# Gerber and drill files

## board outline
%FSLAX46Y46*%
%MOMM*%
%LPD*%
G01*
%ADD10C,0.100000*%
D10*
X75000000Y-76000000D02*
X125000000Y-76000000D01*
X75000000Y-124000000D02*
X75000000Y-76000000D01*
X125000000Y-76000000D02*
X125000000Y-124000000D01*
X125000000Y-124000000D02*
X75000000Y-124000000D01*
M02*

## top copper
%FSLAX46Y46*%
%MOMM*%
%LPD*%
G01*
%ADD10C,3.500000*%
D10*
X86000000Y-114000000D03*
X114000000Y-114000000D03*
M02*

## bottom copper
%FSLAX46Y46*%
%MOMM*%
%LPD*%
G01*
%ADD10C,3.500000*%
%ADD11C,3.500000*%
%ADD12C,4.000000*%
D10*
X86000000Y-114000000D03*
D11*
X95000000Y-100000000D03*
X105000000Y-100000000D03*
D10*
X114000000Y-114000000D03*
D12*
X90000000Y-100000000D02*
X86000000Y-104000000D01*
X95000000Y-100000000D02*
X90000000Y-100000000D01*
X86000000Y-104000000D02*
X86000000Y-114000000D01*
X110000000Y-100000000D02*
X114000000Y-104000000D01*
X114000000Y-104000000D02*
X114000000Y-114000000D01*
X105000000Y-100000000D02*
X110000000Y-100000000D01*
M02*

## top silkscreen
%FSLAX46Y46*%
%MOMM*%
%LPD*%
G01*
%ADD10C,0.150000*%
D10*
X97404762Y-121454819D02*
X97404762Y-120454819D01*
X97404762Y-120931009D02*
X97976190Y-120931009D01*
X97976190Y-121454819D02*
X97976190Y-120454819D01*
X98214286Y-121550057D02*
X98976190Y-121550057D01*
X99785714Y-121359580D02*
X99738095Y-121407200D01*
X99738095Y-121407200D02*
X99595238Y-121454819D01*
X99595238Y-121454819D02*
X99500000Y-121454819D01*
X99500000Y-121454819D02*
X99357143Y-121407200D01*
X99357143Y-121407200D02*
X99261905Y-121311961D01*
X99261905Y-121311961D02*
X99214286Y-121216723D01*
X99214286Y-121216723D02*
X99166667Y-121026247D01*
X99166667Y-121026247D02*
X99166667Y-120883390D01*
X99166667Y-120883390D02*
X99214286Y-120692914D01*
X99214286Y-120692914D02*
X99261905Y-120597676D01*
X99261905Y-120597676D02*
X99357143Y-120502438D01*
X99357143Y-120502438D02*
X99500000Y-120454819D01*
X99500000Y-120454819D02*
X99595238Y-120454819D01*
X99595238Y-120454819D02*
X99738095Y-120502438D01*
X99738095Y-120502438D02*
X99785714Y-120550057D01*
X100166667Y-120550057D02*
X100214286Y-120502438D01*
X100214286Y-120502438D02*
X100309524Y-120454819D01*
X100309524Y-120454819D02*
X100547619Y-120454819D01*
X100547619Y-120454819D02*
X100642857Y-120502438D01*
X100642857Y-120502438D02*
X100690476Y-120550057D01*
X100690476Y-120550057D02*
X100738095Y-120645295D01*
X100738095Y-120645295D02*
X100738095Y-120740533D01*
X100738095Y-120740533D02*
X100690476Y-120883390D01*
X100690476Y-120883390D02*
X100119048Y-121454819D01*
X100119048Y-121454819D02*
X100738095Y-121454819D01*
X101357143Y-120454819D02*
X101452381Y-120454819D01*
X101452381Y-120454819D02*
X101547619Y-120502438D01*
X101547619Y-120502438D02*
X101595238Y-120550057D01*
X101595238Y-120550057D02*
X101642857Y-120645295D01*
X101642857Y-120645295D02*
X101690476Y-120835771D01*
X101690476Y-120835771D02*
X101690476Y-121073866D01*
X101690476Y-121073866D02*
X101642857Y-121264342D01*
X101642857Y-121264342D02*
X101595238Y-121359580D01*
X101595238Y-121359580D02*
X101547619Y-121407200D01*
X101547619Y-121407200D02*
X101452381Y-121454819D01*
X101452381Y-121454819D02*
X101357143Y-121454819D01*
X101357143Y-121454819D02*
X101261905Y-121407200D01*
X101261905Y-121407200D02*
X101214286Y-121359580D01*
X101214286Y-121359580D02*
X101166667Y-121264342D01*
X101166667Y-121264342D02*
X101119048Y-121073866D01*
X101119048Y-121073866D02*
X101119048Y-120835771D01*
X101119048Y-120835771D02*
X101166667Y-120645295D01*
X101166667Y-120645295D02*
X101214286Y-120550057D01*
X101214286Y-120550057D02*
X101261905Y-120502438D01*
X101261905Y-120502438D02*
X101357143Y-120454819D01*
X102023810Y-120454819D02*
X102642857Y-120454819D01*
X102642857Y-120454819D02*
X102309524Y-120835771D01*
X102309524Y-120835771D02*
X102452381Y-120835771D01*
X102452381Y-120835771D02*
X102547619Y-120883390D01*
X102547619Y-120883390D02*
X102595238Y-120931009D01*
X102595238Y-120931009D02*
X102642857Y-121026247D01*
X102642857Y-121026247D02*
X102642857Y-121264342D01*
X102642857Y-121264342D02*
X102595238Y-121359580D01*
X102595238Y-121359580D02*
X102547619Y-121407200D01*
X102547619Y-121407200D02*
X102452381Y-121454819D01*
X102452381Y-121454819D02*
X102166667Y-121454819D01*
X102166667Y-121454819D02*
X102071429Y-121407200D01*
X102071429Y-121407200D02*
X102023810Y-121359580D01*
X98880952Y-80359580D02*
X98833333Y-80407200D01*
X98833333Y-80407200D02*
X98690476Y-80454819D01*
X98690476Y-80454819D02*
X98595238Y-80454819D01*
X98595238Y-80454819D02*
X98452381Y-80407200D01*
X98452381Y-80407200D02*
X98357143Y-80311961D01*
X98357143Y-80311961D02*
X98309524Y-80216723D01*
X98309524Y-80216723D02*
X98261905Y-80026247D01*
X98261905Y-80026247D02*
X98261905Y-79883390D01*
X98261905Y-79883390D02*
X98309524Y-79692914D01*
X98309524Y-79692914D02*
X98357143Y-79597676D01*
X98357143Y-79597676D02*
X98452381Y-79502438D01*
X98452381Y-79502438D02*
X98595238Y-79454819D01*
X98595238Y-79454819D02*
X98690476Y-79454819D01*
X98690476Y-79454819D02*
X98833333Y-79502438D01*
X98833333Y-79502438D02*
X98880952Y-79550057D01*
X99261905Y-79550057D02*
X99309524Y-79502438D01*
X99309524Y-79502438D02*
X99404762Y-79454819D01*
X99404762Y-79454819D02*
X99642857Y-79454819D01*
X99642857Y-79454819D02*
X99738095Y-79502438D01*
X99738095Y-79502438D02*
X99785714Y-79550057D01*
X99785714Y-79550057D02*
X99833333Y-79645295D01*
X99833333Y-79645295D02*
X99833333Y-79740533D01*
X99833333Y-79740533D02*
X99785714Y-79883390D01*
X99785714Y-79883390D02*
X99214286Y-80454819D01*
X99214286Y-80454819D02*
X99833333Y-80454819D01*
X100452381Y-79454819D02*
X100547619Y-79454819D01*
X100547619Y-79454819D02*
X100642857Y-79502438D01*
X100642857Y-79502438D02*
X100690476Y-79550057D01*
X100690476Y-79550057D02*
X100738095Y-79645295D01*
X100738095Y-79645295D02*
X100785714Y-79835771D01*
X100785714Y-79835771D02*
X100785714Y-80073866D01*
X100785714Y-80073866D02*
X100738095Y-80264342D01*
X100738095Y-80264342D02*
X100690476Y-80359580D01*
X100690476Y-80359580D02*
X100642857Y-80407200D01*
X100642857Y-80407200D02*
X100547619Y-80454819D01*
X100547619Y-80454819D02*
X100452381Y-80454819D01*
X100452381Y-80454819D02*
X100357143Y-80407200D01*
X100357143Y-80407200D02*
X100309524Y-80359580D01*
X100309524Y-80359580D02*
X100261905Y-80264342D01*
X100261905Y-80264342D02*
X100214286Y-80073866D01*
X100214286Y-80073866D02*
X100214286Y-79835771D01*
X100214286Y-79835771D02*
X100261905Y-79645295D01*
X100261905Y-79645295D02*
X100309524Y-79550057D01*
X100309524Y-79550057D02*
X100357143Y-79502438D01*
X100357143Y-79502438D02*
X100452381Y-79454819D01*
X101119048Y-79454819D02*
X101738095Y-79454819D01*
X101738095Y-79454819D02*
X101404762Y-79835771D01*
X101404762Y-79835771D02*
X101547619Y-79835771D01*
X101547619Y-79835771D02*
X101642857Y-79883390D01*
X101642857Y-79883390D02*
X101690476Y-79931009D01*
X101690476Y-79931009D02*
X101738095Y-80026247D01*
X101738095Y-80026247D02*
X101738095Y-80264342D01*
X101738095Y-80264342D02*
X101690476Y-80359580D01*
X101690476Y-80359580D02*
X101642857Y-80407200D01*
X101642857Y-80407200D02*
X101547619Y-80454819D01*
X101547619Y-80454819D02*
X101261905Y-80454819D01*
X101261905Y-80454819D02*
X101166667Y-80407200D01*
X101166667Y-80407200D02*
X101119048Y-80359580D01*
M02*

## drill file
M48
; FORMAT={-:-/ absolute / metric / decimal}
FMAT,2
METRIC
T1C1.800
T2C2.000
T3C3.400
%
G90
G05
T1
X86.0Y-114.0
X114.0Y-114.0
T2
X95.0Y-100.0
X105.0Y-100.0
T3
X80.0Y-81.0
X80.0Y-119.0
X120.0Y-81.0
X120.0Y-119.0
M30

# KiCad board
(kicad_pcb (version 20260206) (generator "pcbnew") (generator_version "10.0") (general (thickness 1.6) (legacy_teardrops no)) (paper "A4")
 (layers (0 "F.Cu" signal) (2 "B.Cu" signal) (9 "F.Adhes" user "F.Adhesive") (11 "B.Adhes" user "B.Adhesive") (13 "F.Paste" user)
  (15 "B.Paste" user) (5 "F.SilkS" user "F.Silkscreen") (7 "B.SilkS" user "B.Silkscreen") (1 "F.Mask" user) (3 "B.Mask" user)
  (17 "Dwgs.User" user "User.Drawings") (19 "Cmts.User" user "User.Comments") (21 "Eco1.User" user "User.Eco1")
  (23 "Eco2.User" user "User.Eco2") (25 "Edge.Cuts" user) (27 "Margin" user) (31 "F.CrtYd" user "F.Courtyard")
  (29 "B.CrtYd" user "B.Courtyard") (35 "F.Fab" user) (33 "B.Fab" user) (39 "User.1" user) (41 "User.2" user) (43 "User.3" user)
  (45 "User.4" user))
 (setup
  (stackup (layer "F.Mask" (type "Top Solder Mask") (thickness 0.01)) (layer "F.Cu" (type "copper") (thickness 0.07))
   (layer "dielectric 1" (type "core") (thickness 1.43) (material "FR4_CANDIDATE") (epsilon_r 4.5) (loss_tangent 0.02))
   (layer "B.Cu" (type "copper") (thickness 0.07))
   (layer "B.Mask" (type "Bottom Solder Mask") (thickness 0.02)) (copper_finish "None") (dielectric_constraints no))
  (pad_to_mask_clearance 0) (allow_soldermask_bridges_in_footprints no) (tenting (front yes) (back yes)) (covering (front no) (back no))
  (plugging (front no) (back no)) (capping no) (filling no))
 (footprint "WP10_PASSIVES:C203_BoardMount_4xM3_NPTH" (layer "F.Cu") (at 100 100)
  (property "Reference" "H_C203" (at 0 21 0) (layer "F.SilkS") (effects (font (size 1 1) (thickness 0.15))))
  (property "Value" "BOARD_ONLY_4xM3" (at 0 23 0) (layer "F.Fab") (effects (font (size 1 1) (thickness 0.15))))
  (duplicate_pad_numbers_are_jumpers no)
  (pad "" np_thru_hole circle (at -20 -19) (size 3.4 3.4) (drill 3.4) (layers "*.Cu" "*.Mask"))
  (pad "" np_thru_hole circle (at -20 19) (size 3.4 3.4) (drill 3.4) (layers "*.Cu" "*.Mask"))
  (pad "" np_thru_hole circle (at 20 -19) (size 3.4 3.4) (drill 3.4) (layers "*.Cu" "*.Mask"))
  (pad "" np_thru_hole circle (at 20 19) (size 3.4 3.4) (drill 3.4) (layers "*.Cu" "*.Mask")))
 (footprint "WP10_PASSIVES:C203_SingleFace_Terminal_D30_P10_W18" (layer "F.Cu") (at 100 100)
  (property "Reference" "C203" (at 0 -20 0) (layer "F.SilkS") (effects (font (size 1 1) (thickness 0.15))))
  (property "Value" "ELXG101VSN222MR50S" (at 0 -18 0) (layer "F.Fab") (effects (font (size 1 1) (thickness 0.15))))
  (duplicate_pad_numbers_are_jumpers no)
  (pad "" np_thru_hole circle (at -5 0) (size 2 2) (drill 2) (layers "*.Cu" "F.Mask"))
  (pad "" np_thru_hole circle (at 5 0) (size 2 2) (drill 2) (layers "*.Cu" "F.Mask"))
  (pad "1" thru_hole circle (at -14 14) (size 3.5 3.5) (drill 1.8) (layers "*.Cu" "*.Mask") (remove_unused_layers no)
   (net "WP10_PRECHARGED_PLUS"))
  (pad "1" smd circle (at -5 0) (size 3.5 3.5) (layers "B.Cu" "B.Mask") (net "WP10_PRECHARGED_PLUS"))
  (pad "2" smd circle (at 5 0) (size 3.5 3.5) (layers "B.Cu" "B.Mask") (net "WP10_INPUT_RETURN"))
  (pad "2" thru_hole circle (at 14 14) (size 3.5 3.5) (drill 1.8) (layers "*.Cu" "*.Mask") (remove_unused_layers no)
   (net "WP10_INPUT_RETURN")))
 (gr_line (start 75 76) (end 125 76) (stroke (width 0.1) (type default)) (layer "Edge.Cuts"))
 (gr_line (start 75 124) (end 75 76) (stroke (width 0.1) (type default)) (layer "Edge.Cuts"))
 (gr_line (start 125 76) (end 125 124) (stroke (width 0.1) (type default)) (layer "Edge.Cuts"))
 (gr_line (start 125 124) (end 75 124) (stroke (width 0.1) (type default)) (layer "Edge.Cuts"))
 (segment (start 90 100) (end 86 104) (width 4) (layer "B.Cu") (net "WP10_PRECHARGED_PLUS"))
 (segment (start 95 100) (end 90 100) (width 4) (layer "B.Cu") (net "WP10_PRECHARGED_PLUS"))
 (segment (start 86 104) (end 86 114) (width 4) (layer "B.Cu") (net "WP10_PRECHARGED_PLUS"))
 (segment (start 110 100) (end 114 104) (width 4) (layer "B.Cu") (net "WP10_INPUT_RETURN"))
 (segment (start 114 104) (end 114 114) (width 4) (layer "B.Cu") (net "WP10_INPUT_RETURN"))
 (segment (start 105 100) (end 110 100) (width 4) (layer "B.Cu") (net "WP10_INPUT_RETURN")))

